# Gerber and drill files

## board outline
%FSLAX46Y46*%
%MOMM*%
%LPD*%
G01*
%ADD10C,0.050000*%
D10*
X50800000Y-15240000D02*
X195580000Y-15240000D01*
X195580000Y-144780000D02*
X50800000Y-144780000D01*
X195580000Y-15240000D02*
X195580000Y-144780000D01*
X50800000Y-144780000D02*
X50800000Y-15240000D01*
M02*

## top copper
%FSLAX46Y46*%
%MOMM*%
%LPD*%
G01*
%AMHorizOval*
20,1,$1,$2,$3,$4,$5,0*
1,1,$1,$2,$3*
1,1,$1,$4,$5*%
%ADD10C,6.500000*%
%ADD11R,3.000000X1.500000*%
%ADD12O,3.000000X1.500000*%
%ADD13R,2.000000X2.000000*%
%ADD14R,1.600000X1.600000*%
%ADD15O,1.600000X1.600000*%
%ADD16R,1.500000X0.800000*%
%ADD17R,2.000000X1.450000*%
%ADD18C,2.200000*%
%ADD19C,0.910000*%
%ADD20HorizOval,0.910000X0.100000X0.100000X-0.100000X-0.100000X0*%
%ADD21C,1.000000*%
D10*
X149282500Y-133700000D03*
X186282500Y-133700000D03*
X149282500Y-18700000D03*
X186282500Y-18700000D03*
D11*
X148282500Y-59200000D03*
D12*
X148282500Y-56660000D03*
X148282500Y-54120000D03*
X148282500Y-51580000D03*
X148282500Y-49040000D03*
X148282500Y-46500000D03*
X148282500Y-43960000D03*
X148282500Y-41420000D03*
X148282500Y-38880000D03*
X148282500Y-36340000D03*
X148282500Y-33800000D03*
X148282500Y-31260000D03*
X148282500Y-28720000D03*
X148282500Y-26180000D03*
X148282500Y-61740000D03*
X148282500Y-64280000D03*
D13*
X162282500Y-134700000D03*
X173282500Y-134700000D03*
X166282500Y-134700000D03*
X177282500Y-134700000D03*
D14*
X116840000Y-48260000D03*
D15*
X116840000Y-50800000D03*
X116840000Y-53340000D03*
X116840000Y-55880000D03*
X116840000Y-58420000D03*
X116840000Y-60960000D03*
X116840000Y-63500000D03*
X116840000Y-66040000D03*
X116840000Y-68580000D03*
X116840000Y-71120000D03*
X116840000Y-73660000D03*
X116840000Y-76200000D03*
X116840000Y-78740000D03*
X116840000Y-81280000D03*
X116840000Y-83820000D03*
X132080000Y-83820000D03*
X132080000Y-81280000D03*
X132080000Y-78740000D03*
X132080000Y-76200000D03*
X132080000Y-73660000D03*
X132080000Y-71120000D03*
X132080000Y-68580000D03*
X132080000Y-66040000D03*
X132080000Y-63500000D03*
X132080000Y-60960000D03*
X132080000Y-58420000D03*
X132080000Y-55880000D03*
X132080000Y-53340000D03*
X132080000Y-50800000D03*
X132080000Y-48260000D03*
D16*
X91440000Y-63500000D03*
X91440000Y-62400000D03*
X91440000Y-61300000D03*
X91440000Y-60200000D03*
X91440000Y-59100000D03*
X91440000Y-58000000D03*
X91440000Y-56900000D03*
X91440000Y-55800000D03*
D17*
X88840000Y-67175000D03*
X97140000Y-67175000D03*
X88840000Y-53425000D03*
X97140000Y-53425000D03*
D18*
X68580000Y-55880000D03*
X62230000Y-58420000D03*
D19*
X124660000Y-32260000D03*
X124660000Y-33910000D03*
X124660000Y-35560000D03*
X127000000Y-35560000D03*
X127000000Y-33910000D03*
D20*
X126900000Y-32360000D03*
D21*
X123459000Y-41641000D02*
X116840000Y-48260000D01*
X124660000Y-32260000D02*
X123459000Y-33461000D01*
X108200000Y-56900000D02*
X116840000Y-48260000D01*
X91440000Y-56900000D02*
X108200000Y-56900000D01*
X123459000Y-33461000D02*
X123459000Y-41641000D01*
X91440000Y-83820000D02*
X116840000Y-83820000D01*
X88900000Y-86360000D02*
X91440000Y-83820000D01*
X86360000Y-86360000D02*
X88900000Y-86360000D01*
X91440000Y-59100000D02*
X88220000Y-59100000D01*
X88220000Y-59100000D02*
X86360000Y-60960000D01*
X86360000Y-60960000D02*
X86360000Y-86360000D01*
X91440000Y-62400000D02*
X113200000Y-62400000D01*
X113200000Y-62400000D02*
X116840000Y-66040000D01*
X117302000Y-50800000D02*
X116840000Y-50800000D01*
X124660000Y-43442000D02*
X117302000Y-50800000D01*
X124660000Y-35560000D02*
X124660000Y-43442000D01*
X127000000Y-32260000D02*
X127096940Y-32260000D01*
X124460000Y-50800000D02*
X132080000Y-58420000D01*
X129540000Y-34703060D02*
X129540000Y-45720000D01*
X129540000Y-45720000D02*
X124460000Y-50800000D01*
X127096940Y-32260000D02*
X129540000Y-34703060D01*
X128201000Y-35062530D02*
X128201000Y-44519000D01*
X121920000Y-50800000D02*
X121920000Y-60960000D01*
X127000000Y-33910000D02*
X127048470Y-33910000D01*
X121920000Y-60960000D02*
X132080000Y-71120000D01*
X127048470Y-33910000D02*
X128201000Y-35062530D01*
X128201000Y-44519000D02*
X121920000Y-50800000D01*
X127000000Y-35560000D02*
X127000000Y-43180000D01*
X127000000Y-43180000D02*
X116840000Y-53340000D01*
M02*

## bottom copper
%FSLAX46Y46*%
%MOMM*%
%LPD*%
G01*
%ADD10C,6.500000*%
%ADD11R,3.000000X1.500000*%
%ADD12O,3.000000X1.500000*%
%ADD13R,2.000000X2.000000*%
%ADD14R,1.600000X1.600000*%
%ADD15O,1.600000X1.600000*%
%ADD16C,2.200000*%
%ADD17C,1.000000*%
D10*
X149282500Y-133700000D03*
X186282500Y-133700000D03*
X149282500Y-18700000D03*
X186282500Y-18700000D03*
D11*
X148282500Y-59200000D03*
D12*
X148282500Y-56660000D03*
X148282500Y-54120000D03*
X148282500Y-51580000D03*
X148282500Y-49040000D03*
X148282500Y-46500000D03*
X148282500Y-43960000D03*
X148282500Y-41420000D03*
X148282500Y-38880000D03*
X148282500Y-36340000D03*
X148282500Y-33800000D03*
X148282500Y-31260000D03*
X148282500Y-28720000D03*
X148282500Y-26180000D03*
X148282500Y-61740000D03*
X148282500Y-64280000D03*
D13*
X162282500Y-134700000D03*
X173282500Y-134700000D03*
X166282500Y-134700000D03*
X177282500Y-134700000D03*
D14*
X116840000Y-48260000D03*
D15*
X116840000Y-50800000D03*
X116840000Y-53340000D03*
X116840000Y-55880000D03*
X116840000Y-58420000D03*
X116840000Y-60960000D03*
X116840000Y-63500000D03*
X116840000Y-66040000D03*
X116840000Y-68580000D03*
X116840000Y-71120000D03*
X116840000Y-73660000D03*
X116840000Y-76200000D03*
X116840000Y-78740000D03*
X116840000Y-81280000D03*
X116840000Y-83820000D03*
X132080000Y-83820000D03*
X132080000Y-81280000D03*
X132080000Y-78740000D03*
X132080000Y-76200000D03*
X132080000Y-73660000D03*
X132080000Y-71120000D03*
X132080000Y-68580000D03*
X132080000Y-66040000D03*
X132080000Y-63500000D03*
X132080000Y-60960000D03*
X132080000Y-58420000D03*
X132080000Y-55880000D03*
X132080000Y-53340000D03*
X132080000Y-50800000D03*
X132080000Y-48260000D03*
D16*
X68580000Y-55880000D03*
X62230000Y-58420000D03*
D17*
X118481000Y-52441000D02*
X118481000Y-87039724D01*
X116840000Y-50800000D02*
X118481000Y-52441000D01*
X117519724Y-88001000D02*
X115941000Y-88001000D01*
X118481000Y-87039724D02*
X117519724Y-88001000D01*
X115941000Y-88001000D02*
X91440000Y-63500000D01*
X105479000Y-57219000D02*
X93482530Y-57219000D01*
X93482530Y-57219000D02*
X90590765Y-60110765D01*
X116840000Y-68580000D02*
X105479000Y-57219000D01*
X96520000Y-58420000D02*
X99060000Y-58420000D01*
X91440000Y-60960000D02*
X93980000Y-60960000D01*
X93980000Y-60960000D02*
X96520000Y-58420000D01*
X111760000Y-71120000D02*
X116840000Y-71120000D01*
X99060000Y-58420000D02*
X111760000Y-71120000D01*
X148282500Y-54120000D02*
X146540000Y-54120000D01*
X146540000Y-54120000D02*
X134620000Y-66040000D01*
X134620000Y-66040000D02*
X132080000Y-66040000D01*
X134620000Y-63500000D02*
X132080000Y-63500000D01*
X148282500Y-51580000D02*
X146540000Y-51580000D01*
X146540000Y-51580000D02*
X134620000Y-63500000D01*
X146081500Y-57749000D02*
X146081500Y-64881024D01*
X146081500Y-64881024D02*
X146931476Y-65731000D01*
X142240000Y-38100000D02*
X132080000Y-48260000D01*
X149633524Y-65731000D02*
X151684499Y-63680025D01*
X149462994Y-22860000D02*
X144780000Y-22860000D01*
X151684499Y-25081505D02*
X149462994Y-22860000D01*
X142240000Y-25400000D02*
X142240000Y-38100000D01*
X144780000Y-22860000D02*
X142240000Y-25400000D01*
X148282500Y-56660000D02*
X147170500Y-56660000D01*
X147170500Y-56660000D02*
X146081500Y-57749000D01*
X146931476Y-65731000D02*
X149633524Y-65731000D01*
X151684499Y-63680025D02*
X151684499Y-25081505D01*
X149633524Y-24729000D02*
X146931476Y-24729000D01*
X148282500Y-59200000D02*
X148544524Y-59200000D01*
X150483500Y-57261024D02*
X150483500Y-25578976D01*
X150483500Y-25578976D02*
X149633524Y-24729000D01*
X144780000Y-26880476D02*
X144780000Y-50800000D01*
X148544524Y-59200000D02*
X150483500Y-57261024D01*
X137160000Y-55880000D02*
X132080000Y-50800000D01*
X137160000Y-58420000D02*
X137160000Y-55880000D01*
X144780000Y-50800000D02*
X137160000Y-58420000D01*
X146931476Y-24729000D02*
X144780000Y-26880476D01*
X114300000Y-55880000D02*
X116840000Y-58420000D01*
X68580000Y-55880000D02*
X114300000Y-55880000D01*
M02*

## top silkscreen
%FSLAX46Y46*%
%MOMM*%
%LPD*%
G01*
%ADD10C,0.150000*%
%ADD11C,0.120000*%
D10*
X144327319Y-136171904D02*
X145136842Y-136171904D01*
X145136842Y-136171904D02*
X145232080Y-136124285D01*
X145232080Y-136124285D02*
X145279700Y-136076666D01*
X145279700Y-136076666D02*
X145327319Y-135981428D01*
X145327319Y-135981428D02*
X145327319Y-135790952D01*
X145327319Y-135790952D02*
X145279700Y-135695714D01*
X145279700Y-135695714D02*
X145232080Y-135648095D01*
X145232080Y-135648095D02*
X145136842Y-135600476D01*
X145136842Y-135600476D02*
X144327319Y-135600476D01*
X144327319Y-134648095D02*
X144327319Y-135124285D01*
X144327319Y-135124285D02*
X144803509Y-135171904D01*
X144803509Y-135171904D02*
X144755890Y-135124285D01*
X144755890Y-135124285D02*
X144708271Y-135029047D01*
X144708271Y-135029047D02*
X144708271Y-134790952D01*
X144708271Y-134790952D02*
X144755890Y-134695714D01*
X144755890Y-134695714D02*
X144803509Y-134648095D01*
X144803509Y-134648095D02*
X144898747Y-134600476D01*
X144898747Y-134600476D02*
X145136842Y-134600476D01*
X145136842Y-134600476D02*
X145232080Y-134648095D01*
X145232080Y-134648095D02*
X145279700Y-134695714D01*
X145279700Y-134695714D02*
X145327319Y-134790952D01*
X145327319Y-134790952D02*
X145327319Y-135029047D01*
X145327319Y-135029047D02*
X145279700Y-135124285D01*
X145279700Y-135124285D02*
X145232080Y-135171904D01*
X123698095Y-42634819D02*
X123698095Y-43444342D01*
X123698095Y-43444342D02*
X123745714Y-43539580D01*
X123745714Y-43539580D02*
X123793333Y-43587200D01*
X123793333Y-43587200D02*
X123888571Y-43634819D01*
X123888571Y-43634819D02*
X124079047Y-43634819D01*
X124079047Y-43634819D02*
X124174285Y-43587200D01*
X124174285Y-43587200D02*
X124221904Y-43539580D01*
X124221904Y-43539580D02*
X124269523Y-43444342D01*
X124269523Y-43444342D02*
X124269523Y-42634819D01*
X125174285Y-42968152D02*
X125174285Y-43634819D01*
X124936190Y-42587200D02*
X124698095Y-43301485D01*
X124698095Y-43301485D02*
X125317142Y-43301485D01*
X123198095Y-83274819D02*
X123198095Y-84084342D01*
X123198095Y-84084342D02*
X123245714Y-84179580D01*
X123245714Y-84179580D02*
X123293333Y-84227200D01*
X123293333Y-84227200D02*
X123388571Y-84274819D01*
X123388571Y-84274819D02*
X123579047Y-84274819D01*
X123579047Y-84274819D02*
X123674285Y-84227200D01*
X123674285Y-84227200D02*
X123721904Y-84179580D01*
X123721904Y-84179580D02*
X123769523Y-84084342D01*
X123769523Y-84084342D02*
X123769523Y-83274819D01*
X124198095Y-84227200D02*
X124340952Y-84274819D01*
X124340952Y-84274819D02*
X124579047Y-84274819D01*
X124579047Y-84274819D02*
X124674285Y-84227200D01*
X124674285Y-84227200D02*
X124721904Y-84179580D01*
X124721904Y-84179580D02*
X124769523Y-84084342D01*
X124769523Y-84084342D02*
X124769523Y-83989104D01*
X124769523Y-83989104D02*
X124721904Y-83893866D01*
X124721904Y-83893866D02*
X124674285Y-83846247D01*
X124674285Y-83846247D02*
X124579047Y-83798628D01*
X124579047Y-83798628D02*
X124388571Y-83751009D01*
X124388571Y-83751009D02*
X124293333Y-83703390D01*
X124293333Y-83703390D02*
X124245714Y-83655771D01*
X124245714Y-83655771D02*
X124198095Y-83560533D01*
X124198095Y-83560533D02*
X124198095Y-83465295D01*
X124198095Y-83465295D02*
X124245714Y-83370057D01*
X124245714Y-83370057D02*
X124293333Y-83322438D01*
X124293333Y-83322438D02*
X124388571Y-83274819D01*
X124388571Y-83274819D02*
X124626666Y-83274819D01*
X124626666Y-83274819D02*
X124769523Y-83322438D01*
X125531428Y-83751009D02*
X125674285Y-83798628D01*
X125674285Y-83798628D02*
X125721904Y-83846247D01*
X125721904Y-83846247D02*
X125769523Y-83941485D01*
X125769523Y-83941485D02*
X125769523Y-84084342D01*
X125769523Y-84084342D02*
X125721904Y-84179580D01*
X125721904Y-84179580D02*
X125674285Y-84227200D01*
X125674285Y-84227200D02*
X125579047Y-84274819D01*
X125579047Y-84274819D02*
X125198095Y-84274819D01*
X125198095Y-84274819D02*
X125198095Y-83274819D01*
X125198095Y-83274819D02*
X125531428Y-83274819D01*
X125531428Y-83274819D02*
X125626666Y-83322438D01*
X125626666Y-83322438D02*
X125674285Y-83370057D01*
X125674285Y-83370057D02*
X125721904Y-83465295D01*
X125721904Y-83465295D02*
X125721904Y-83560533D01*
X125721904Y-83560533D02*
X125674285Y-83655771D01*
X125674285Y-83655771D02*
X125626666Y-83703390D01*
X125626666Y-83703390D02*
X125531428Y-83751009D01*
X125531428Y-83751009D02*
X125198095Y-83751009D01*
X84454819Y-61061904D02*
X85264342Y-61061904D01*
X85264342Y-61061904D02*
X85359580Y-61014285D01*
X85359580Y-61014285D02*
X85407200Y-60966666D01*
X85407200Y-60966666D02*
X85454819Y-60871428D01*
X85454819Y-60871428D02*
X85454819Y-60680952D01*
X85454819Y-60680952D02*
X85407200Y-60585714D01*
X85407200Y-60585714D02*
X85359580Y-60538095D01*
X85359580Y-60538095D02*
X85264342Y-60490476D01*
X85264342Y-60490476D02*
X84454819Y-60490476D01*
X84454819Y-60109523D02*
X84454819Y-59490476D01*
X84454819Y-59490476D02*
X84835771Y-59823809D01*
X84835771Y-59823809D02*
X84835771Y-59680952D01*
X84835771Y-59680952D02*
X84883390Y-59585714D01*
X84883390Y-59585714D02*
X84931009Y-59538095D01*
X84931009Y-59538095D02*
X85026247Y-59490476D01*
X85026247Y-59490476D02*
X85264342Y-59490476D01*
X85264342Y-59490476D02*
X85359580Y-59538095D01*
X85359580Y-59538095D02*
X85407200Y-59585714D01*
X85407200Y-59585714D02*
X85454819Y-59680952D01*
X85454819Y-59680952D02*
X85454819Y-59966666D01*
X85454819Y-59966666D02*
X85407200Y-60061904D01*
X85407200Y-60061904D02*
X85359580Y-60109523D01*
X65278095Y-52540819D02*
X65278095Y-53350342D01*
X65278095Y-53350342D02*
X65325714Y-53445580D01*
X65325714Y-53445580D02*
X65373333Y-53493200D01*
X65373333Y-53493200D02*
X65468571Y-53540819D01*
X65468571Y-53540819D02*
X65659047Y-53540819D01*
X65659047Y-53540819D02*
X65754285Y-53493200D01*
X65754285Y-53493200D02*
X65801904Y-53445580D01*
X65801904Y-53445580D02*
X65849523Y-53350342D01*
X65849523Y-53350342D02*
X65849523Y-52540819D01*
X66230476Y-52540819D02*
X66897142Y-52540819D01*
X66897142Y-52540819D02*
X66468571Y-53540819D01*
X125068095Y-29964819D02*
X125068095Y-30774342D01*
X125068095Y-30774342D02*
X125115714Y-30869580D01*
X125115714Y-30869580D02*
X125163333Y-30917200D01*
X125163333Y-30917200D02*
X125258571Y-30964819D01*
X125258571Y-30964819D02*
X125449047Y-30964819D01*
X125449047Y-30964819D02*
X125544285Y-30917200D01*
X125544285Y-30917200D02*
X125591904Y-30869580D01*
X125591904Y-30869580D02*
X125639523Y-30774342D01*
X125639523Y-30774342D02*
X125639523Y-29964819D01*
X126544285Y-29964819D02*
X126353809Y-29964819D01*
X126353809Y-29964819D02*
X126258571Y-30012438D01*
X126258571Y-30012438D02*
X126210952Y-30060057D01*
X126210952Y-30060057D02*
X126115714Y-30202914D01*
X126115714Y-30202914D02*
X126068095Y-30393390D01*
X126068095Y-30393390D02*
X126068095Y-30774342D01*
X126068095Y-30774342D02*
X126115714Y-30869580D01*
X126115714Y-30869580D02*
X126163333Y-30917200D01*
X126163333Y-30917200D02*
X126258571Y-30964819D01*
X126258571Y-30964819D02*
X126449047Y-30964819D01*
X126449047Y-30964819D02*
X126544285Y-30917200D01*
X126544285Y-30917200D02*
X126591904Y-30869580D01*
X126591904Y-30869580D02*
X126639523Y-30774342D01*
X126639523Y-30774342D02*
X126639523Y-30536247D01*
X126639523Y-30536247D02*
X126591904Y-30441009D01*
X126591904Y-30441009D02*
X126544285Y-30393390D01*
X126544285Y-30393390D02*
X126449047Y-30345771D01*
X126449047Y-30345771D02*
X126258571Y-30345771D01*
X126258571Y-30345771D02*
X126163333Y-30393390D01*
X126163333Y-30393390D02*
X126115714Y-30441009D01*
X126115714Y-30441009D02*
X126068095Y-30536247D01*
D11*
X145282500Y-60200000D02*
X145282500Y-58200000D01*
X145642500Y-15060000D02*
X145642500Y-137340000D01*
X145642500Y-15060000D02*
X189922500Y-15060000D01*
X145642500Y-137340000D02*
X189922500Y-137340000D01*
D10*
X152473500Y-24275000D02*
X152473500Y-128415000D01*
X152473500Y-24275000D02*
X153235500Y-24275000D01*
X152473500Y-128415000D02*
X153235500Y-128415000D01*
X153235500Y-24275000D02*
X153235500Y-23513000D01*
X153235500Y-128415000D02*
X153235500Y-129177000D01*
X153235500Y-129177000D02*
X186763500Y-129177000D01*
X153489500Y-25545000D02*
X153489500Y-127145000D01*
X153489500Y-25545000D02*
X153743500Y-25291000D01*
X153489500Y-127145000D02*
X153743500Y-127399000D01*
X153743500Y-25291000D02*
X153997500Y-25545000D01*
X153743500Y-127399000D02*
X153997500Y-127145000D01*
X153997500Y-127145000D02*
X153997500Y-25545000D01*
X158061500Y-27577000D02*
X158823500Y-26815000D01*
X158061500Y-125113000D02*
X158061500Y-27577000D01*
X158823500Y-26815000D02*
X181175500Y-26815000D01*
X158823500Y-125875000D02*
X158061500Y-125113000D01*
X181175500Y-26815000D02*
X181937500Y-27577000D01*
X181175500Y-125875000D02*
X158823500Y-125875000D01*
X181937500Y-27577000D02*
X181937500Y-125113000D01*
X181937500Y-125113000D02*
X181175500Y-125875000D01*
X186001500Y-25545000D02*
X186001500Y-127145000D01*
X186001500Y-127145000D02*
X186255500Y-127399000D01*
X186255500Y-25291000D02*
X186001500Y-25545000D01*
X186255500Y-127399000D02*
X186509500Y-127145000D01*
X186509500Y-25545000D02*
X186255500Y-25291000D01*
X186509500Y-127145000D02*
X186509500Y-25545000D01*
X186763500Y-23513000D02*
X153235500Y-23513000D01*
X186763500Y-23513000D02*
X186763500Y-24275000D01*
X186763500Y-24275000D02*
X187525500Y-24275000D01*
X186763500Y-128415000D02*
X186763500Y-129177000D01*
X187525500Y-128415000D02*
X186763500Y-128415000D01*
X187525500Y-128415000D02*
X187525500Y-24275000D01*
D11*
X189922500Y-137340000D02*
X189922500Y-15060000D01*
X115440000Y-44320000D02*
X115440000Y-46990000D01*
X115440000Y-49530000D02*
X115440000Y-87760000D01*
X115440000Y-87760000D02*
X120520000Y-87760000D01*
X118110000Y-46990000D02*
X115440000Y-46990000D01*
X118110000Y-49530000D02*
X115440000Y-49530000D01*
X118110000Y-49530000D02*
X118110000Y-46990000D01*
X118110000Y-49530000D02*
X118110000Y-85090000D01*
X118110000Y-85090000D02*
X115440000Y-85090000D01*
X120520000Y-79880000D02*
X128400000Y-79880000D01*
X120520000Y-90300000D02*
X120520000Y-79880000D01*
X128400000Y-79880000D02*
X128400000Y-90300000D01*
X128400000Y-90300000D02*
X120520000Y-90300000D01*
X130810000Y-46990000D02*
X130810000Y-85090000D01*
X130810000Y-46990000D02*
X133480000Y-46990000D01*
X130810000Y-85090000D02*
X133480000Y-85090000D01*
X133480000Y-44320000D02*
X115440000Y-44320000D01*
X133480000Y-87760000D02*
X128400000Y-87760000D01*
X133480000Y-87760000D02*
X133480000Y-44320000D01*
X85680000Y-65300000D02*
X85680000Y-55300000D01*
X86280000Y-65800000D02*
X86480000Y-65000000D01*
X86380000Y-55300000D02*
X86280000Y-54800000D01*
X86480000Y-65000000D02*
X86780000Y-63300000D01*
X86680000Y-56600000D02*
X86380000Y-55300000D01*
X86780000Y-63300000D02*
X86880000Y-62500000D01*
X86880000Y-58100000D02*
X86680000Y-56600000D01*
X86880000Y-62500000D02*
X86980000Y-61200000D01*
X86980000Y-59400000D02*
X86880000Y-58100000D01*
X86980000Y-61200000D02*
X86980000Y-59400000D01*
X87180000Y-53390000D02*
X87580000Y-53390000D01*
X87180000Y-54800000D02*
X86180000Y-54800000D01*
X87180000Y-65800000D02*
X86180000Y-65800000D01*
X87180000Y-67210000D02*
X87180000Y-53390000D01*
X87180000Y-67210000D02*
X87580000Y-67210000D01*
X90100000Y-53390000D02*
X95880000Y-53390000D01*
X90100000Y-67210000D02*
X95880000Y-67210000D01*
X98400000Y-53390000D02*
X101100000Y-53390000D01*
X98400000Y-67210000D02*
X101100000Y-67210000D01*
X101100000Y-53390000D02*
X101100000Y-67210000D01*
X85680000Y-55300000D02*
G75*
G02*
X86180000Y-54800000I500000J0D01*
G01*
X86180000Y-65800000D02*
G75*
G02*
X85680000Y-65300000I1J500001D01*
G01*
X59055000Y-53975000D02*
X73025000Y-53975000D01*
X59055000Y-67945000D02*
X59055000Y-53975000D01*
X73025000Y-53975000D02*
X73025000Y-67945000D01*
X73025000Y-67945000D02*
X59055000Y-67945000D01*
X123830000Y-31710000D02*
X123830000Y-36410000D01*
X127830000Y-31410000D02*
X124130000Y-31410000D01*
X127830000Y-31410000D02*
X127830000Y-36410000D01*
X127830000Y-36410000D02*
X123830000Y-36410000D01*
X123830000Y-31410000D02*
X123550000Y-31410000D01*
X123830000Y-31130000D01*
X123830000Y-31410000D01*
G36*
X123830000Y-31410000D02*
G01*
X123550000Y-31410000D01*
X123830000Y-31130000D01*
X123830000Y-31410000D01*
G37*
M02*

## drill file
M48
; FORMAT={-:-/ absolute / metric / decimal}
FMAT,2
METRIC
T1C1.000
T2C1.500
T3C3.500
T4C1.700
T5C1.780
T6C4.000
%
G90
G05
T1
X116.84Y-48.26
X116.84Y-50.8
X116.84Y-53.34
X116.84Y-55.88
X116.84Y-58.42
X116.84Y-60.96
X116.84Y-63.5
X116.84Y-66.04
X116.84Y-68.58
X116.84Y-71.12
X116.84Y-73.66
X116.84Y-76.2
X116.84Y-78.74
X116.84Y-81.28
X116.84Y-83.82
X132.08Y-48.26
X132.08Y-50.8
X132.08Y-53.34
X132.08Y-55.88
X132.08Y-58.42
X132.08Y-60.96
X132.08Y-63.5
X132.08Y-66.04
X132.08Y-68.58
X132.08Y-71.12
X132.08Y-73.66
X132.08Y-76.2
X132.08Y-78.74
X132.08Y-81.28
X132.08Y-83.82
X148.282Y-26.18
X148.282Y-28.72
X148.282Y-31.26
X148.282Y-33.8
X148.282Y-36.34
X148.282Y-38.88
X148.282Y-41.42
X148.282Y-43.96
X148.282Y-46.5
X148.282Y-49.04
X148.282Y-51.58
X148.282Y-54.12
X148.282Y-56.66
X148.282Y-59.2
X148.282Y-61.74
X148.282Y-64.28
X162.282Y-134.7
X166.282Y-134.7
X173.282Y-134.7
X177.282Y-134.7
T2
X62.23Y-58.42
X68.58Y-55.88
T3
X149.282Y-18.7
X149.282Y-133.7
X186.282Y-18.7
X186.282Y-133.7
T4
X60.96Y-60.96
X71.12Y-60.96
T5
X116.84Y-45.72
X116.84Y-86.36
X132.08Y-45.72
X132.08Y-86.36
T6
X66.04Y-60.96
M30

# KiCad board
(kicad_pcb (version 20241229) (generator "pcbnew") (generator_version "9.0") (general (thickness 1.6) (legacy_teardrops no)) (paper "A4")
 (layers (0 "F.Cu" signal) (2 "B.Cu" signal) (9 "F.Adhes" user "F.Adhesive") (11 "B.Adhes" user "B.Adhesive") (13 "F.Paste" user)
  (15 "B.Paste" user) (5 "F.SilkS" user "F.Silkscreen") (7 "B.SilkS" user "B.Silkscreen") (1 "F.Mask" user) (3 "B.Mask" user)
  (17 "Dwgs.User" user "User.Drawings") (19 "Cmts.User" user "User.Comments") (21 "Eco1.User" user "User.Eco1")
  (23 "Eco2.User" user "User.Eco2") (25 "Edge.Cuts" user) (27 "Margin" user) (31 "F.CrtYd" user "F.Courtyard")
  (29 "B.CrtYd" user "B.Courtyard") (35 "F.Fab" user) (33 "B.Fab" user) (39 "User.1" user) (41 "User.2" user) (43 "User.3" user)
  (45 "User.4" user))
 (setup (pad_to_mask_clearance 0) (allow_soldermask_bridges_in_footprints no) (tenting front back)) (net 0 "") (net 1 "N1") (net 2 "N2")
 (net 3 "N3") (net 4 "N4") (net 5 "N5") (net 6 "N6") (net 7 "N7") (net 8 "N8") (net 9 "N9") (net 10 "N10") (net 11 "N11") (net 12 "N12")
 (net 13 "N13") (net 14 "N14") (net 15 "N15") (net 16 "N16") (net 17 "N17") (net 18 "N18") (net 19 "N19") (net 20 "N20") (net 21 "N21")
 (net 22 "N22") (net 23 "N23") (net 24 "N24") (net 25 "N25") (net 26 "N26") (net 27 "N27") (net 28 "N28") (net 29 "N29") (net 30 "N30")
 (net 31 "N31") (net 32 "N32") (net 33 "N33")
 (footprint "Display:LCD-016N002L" (layer "F.Cu") (at 148.2825 59.2 90)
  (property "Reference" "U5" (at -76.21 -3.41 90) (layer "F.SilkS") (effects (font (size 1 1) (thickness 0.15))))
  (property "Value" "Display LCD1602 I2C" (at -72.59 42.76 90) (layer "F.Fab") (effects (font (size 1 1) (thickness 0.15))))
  (fp_line (start -1 -3) (end 1 -3) (stroke (width 0.12) (type solid)) (layer "F.SilkS"))
  (fp_line (start 44.14 -2.64) (end -78.14 -2.64) (stroke (width 0.12) (type solid)) (layer "F.SilkS"))
  (fp_line (start 44.14 -2.64) (end 44.14 41.64) (stroke (width 0.12) (type solid)) (layer "F.SilkS"))
  (fp_line (start -78.14 -2.64) (end -78.14 41.64) (stroke (width 0.12) (type solid)) (layer "F.SilkS"))
  (fp_line (start 34.925 4.191) (end -69.215 4.191) (stroke (width 0.15) (type solid)) (layer "F.SilkS"))
  (fp_line (start 34.925 4.191) (end 34.925 4.953) (stroke (width 0.15) (type solid)) (layer "F.SilkS"))
  (fp_line (start -69.215 4.191) (end -69.215 4.953) (stroke (width 0.15) (type solid)) (layer "F.SilkS"))
  (fp_line (start 34.925 4.953) (end 35.687 4.953) (stroke (width 0.15) (type solid)) (layer "F.SilkS"))
  (fp_line (start -69.215 4.953) (end -69.977 4.953) (stroke (width 0.15) (type solid)) (layer "F.SilkS"))
  (fp_line (start -69.977 4.953) (end -69.977 38.481) (stroke (width 0.15) (type solid)) (layer "F.SilkS"))
  (fp_line (start 33.655 5.207) (end -67.945 5.207) (stroke (width 0.15) (type solid)) (layer "F.SilkS"))
  (fp_line (start 33.655 5.207) (end 33.909 5.461) (stroke (width 0.15) (type solid)) (layer "F.SilkS"))
  (fp_line (start -67.945 5.207) (end -68.199 5.461) (stroke (width 0.15) (type solid)) (layer "F.SilkS"))
  (fp_line (start 33.909 5.461) (end 33.655 5.715) (stroke (width 0.15) (type solid)) (layer "F.SilkS"))
  (fp_line (start -68.199 5.461) (end -67.945 5.715) (stroke (width 0.15) (type solid)) (layer "F.SilkS"))
  (fp_line (start -67.945 5.715) (end 33.655 5.715) (stroke (width 0.15) (type solid)) (layer "F.SilkS"))
  (fp_line (start 31.623 9.779) (end 32.385 10.541) (stroke (width 0.15) (type solid)) (layer "F.SilkS"))
  (fp_line (start -65.913 9.779) (end 31.623 9.779) (stroke (width 0.15) (type solid)) (layer "F.SilkS"))
  (fp_line (start 32.385 10.541) (end 32.385 32.893) (stroke (width 0.15) (type solid)) (layer "F.SilkS"))
  (fp_line (start -66.675 10.541) (end -65.913 9.779) (stroke (width 0.15) (type solid)) (layer "F.SilkS"))
  (fp_line (start 32.385 32.893) (end 31.623 33.655) (stroke (width 0.15) (type solid)) (layer "F.SilkS"))
  (fp_line (start -66.675 32.893) (end -66.675 10.541) (stroke (width 0.15) (type solid)) (layer "F.SilkS"))
  (fp_line (start 31.623 33.655) (end -65.913 33.655) (stroke (width 0.15) (type solid)) (layer "F.SilkS"))
  (fp_line (start -65.913 33.655) (end -66.675 32.893) (stroke (width 0.15) (type solid)) (layer "F.SilkS"))
  (fp_line (start 33.655 37.719) (end -67.945 37.719) (stroke (width 0.15) (type solid)) (layer "F.SilkS"))
  (fp_line (start -67.945 37.719) (end -68.199 37.973) (stroke (width 0.15) (type solid)) (layer "F.SilkS"))
  (fp_line (start 33.909 37.973) (end 33.655 37.719) (stroke (width 0.15) (type solid)) (layer "F.SilkS"))
  (fp_line (start -68.199 37.973) (end -67.945 38.227) (stroke (width 0.15) (type solid)) (layer "F.SilkS"))
  (fp_line (start 33.655 38.227) (end 33.909 37.973) (stroke (width 0.15) (type solid)) (layer "F.SilkS"))
  (fp_line (start -67.945 38.227) (end 33.655 38.227) (stroke (width 0.15) (type solid)) (layer "F.SilkS"))
  (fp_line (start 35.687 38.481) (end 35.687 4.953) (stroke (width 0.15) (type solid)) (layer "F.SilkS"))
  (fp_line (start 35.687 38.481) (end 34.925 38.481) (stroke (width 0.15) (type solid)) (layer "F.SilkS"))
  (fp_line (start 34.925 38.481) (end 34.925 39.243) (stroke (width 0.15) (type solid)) (layer "F.SilkS"))
  (fp_line (start -69.215 38.481) (end -69.977 38.481) (stroke (width 0.15) (type solid)) (layer "F.SilkS"))
  (fp_line (start -69.215 39.243) (end -69.215 38.481) (stroke (width 0.15) (type solid)) (layer "F.SilkS"))
  (fp_line (start -69.215 39.243) (end 34.925 39.243) (stroke (width 0.15) (type solid)) (layer "F.SilkS"))
  (fp_line (start -78.14 41.64) (end 44.14 41.64) (stroke (width 0.12) (type solid)) (layer "F.SilkS"))
  (pad "" thru_hole circle (at -74.5 1 270) (size 6.5 6.5) (drill 3.5) (layers "*.Cu" "*.Mask") (remove_unused_layers no))
  (pad "" thru_hole circle (at -74.5 38 270) (size 6.5 6.5) (drill 3.5) (layers "*.Cu" "*.Mask") (remove_unused_layers no))
  (pad "" thru_hole circle (at 40.5 1 270) (size 6.5 6.5) (drill 3.5) (layers "*.Cu" "*.Mask") (remove_unused_layers no))
  (pad "" thru_hole circle (at 40.5 38 270) (size 6.5 6.5) (drill 3.5) (layers "*.Cu" "*.Mask") (remove_unused_layers no))
  (pad "1" thru_hole rect (at 0 0 270) (size 1.5 3) (drill 1) (layers "*.Cu" "*.Mask") (remove_unused_layers no) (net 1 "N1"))
  (pad "2" thru_hole oval (at 2.54 0 270) (size 1.5 3) (drill 1) (layers "*.Cu" "*.Mask") (remove_unused_layers no) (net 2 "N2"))
  (pad "3" thru_hole oval (at 5.08 0 270) (size 1.5 3) (drill 1) (layers "*.Cu" "*.Mask") (remove_unused_layers no) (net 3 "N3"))
  (pad "4" thru_hole oval (at 7.62 0 270) (size 1.5 3) (drill 1) (layers "*.Cu" "*.Mask") (remove_unused_layers no) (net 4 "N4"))
  (pad "5" thru_hole oval (at 10.16 0 270) (size 1.5 3) (drill 1) (layers "*.Cu" "*.Mask") (remove_unused_layers no))
  (pad "6" thru_hole oval (at 12.7 0 270) (size 1.5 3) (drill 1) (layers "*.Cu" "*.Mask") (remove_unused_layers no))
  (pad "7" thru_hole oval (at 15.24 0 270) (size 1.5 3) (drill 1) (layers "*.Cu" "*.Mask") (remove_unused_layers no))
  (pad "8" thru_hole oval (at 17.78 0 270) (size 1.5 3) (drill 1) (layers "*.Cu" "*.Mask") (remove_unused_layers no))
  (pad "9" thru_hole oval (at 20.32 0 270) (size 1.5 3) (drill 1) (layers "*.Cu" "*.Mask") (remove_unused_layers no))
  (pad "10" thru_hole oval (at 22.86 0 270) (size 1.5 3) (drill 1) (layers "*.Cu" "*.Mask") (remove_unused_layers no))
  (pad "11" thru_hole oval (at 25.4 0 270) (size 1.5 3) (drill 1) (layers "*.Cu" "*.Mask") (remove_unused_layers no))
  (pad "12" thru_hole oval (at 27.94 0 270) (size 1.5 3) (drill 1) (layers "*.Cu" "*.Mask") (remove_unused_layers no))
  (pad "13" thru_hole oval (at 30.48 0 270) (size 1.5 3) (drill 1) (layers "*.Cu" "*.Mask") (remove_unused_layers no))
  (pad "14" thru_hole oval (at 33.02 0 270) (size 1.5 3) (drill 1) (layers "*.Cu" "*.Mask") (remove_unused_layers no))
  (pad "15" thru_hole oval (at -2.54 0 270) (size 1.5 3) (drill 1) (layers "*.Cu" "*.Mask") (remove_unused_layers no))
  (pad "16" thru_hole oval (at -5.08 0 270) (size 1.5 3) (drill 1) (layers "*.Cu" "*.Mask") (remove_unused_layers no))
  (pad "A1" thru_hole rect (at -75.5 14 270) (size 2 2) (drill 1) (layers "*.Cu" "*.Mask") (remove_unused_layers no))
  (pad "A2" thru_hole rect (at -75.5 25 270) (size 2 2) (drill 1) (layers "*.Cu" "*.Mask") (remove_unused_layers no))
  (pad "K1" thru_hole rect (at -75.5 18 270) (size 2 2) (drill 1) (layers "*.Cu" "*.Mask") (remove_unused_layers no))
  (pad "K2" thru_hole rect (at -75.5 29 270) (size 2 2) (drill 1) (layers "*.Cu" "*.Mask") (remove_unused_layers no)))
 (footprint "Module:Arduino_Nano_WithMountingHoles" (layer "F.Cu") (at 116.84 48.26)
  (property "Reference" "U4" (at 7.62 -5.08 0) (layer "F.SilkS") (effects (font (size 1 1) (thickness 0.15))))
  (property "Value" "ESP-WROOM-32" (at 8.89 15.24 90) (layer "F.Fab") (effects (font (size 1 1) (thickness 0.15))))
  (fp_line (start -1.4 -3.94) (end -1.4 -1.27) (stroke (width 0.12) (type solid)) (layer "F.SilkS"))
  (fp_line (start -1.4 1.27) (end -1.4 39.5) (stroke (width 0.12) (type solid)) (layer "F.SilkS"))
  (fp_line (start -1.4 39.5) (end 3.68 39.5) (stroke (width 0.12) (type solid)) (layer "F.SilkS"))
  (fp_line (start 1.27 -1.27) (end -1.4 -1.27) (stroke (width 0.12) (type solid)) (layer "F.SilkS"))
  (fp_line (start 1.27 1.27) (end -1.4 1.27) (stroke (width 0.12) (type solid)) (layer "F.SilkS"))
  (fp_line (start 1.27 1.27) (end 1.27 -1.27) (stroke (width 0.12) (type solid)) (layer "F.SilkS"))
  (fp_line (start 1.27 1.27) (end 1.27 36.83) (stroke (width 0.12) (type solid)) (layer "F.SilkS"))
  (fp_line (start 1.27 36.83) (end -1.4 36.83) (stroke (width 0.12) (type solid)) (layer "F.SilkS"))
  (fp_line (start 3.68 31.62) (end 11.56 31.62) (stroke (width 0.12) (type solid)) (layer "F.SilkS"))
  (fp_line (start 3.68 42.04) (end 3.68 31.62) (stroke (width 0.12) (type solid)) (layer "F.SilkS"))
  (fp_line (start 11.56 31.62) (end 11.56 42.04) (stroke (width 0.12) (type solid)) (layer "F.SilkS"))
  (fp_line (start 11.56 42.04) (end 3.68 42.04) (stroke (width 0.12) (type solid)) (layer "F.SilkS"))
  (fp_line (start 13.97 -1.27) (end 13.97 36.83) (stroke (width 0.12) (type solid)) (layer "F.SilkS"))
  (fp_line (start 13.97 -1.27) (end 16.64 -1.27) (stroke (width 0.12) (type solid)) (layer "F.SilkS"))
  (fp_line (start 13.97 36.83) (end 16.64 36.83) (stroke (width 0.12) (type solid)) (layer "F.SilkS"))
  (fp_line (start 16.64 -3.94) (end -1.4 -3.94) (stroke (width 0.12) (type solid)) (layer "F.SilkS"))
  (fp_line (start 16.64 39.5) (end 11.56 39.5) (stroke (width 0.12) (type solid)) (layer "F.SilkS"))
  (fp_line (start 16.64 39.5) (end 16.64 -3.94) (stroke (width 0.12) (type solid)) (layer "F.SilkS"))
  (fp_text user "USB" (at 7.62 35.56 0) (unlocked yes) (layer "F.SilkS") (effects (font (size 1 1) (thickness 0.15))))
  (pad "" np_thru_hole circle (at 0 -2.54) (size 1.78 1.78) (drill 1.78) (layers "*.Cu" "*.Mask"))
  (pad "" np_thru_hole circle (at 0 38.1) (size 1.78 1.78) (drill 1.78) (layers "*.Cu" "*.Mask"))
  (pad "" np_thru_hole circle (at 15.24 -2.54) (size 1.78 1.78) (drill 1.78) (layers "*.Cu" "*.Mask"))
  (pad "" np_thru_hole circle (at 15.24 38.1) (size 1.78 1.78) (drill 1.78) (layers "*.Cu" "*.Mask"))
  (pad "1" thru_hole rect (at 0 0) (size 1.6 1.6) (drill 1) (layers "*.Cu" "*.Mask") (remove_unused_layers no) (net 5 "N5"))
  (pad "2" thru_hole oval (at 0 2.54) (size 1.6 1.6) (drill 1) (layers "*.Cu" "*.Mask") (remove_unused_layers no) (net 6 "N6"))
  (pad "3" thru_hole oval (at 0 5.08) (size 1.6 1.6) (drill 1) (layers "*.Cu" "*.Mask") (remove_unused_layers no) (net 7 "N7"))
  (pad "4" thru_hole oval (at 0 7.62) (size 1.6 1.6) (drill 1) (layers "*.Cu" "*.Mask") (remove_unused_layers no) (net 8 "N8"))
  (pad "5" thru_hole oval (at 0 10.16) (size 1.6 1.6) (drill 1) (layers "*.Cu" "*.Mask") (remove_unused_layers no) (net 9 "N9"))
  (pad "6" thru_hole oval (at 0 12.7) (size 1.6 1.6) (drill 1) (layers "*.Cu" "*.Mask") (remove_unused_layers no) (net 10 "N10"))
  (pad "7" thru_hole oval (at 0 15.24) (size 1.6 1.6) (drill 1) (layers "*.Cu" "*.Mask") (remove_unused_layers no) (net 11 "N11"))
  (pad "8" thru_hole oval (at 0 17.78) (size 1.6 1.6) (drill 1) (layers "*.Cu" "*.Mask") (remove_unused_layers no) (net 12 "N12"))
  (pad "9" thru_hole oval (at 0 20.32) (size 1.6 1.6) (drill 1) (layers "*.Cu" "*.Mask") (remove_unused_layers no) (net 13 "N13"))
  (pad "10" thru_hole oval (at 0 22.86) (size 1.6 1.6) (drill 1) (layers "*.Cu" "*.Mask") (remove_unused_layers no) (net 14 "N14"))
  (pad "11" thru_hole oval (at 0 25.4) (size 1.6 1.6) (drill 1) (layers "*.Cu" "*.Mask") (remove_unused_layers no) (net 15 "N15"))
  (pad "12" thru_hole oval (at 0 27.94) (size 1.6 1.6) (drill 1) (layers "*.Cu" "*.Mask") (remove_unused_layers no) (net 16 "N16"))
  (pad "13" thru_hole oval (at 0 30.48) (size 1.6 1.6) (drill 1) (layers "*.Cu" "*.Mask") (remove_unused_layers no) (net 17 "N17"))
  (pad "14" thru_hole oval (at 0 33.02) (size 1.6 1.6) (drill 1) (layers "*.Cu" "*.Mask") (remove_unused_layers no) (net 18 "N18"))
  (pad "15" thru_hole oval (at 0 35.56) (size 1.6 1.6) (drill 1) (layers "*.Cu" "*.Mask") (remove_unused_layers no) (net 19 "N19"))
  (pad "16" thru_hole oval (at 15.24 35.56) (size 1.6 1.6) (drill 1) (layers "*.Cu" "*.Mask") (remove_unused_layers no) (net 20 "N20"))
  (pad "17" thru_hole oval (at 15.24 33.02) (size 1.6 1.6) (drill 1) (layers "*.Cu" "*.Mask") (remove_unused_layers no) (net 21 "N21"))
  (pad "18" thru_hole oval (at 15.24 30.48) (size 1.6 1.6) (drill 1) (layers "*.Cu" "*.Mask") (remove_unused_layers no) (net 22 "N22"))
  (pad "19" thru_hole oval (at 15.24 27.94) (size 1.6 1.6) (drill 1) (layers "*.Cu" "*.Mask") (remove_unused_layers no) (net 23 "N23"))
  (pad "20" thru_hole oval (at 15.24 25.4) (size 1.6 1.6) (drill 1) (layers "*.Cu" "*.Mask") (remove_unused_layers no) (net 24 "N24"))
  (pad "21" thru_hole oval (at 15.24 22.86) (size 1.6 1.6) (drill 1) (layers "*.Cu" "*.Mask") (remove_unused_layers no) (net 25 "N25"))
  (pad "22" thru_hole oval (at 15.24 20.32) (size 1.6 1.6) (drill 1) (layers "*.Cu" "*.Mask") (remove_unused_layers no) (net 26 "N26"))
  (pad "23" thru_hole oval (at 15.24 17.78) (size 1.6 1.6) (drill 1) (layers "*.Cu" "*.Mask") (remove_unused_layers no) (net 3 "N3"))
  (pad "24" thru_hole oval (at 15.24 15.24) (size 1.6 1.6) (drill 1) (layers "*.Cu" "*.Mask") (remove_unused_layers no) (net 4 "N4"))
  (pad "25" thru_hole oval (at 15.24 12.7) (size 1.6 1.6) (drill 1) (layers "*.Cu" "*.Mask") (remove_unused_layers no) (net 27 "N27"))
  (pad "26" thru_hole oval (at 15.24 10.16) (size 1.6 1.6) (drill 1) (layers "*.Cu" "*.Mask") (remove_unused_layers no) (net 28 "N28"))
  (pad "27" thru_hole oval (at 15.24 7.62) (size 1.6 1.6) (drill 1) (layers "*.Cu" "*.Mask") (remove_unused_layers no) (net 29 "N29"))
  (pad "28" thru_hole oval (at 15.24 5.08) (size 1.6 1.6) (drill 1) (layers "*.Cu" "*.Mask") (remove_unused_layers no) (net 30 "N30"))
  (pad "29" thru_hole oval (at 15.24 2.54) (size 1.6 1.6) (drill 1) (layers "*.Cu" "*.Mask") (remove_unused_layers no) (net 1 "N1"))
  (pad "30" thru_hole oval (at 15.24 0) (size 1.6 1.6) (drill 1) (layers "*.Cu" "*.Mask") (remove_unused_layers no) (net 2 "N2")))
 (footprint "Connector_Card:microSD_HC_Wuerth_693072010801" (layer "F.Cu") (at 92.99 60.3 90)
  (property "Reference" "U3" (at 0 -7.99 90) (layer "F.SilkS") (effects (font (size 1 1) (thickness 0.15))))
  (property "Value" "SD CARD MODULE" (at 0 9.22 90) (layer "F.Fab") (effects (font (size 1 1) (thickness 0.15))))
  (fp_line (start -5 -7.31) (end 5 -7.31) (stroke (width 0.12) (type solid)) (layer "F.SilkS"))
  (fp_line (start -5.5 -6.71) (end -4.7 -6.51) (stroke (width 0.12) (type solid)) (layer "F.SilkS"))
  (fp_line (start 5 -6.61) (end 5.5 -6.71) (stroke (width 0.12) (type solid)) (layer "F.SilkS"))
  (fp_line (start -4.7 -6.51) (end -3 -6.21) (stroke (width 0.12) (type solid)) (layer "F.SilkS"))
  (fp_line (start 3.7 -6.31) (end 5 -6.61) (stroke (width 0.12) (type solid)) (layer "F.SilkS"))
  (fp_line (start -3 -6.21) (end -2.2 -6.11) (stroke (width 0.12) (type solid)) (layer "F.SilkS"))
  (fp_line (start 2.2 -6.11) (end 3.7 -6.31) (stroke (width 0.12) (type solid)) (layer "F.SilkS"))
  (fp_line (start -2.2 -6.11) (end -0.9 -6.01) (stroke (width 0.12) (type solid)) (layer "F.SilkS"))
  (fp_line (start 0.9 -6.01) (end 2.2 -6.11) (stroke (width 0.12) (type solid)) (layer "F.SilkS"))
  (fp_line (start -0.9 -6.01) (end 0.9 -6.01) (stroke (width 0.12) (type solid)) (layer "F.SilkS"))
  (fp_line (start 6.91 -5.81) (end 6.91 -5.41) (stroke (width 0.12) (type solid)) (layer "F.SilkS"))
  (fp_line (start 5.5 -5.81) (end 5.5 -6.81) (stroke (width 0.12) (type solid)) (layer "F.SilkS"))
  (fp_line (start -5.5 -5.81) (end -5.5 -6.81) (stroke (width 0.12) (type solid)) (layer "F.SilkS"))
  (fp_line (start -6.91 -5.81) (end 6.91 -5.81) (stroke (width 0.12) (type solid)) (layer "F.SilkS"))
  (fp_line (start -6.91 -5.81) (end -6.91 -5.41) (stroke (width 0.12) (type solid)) (layer "F.SilkS"))
  (fp_line (start 6.91 -2.89) (end 6.91 2.89) (stroke (width 0.12) (type solid)) (layer "F.SilkS"))
  (fp_line (start -6.91 -2.89) (end -6.91 2.89) (stroke (width 0.12) (type solid)) (layer "F.SilkS"))
  (fp_line (start 6.91 5.41) (end 6.91 8.11) (stroke (width 0.12) (type solid)) (layer "F.SilkS"))
  (fp_line (start -6.91 5.41) (end -6.91 8.11) (stroke (width 0.12) (type solid)) (layer "F.SilkS"))
  (fp_line (start 6.91 8.11) (end -6.91 8.11) (stroke (width 0.12) (type solid)) (layer "F.SilkS"))
  (fp_arc (start 5 -7.31) (mid 5.353553 -7.163553) (end 5.5 -6.81) (stroke (width 0.12) (type solid)) (layer "F.SilkS"))
  (fp_arc (start -5.5 -6.81) (mid -5.353553 -7.163553) (end -5 -7.31) (stroke (width 0.12) (type solid)) (layer "F.SilkS"))
  (pad "1" smd rect (at -3.2 -1.55 90) (size 0.8 1.5) (layers "F.Cu" "F.Mask" "F.Paste") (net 6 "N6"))
  (pad "2" smd rect (at -2.1 -1.55 90) (size 0.8 1.5) (layers "F.Cu" "F.Mask" "F.Paste") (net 12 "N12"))
  (pad "3" smd rect (at -1 -1.55 90) (size 0.8 1.5) (layers "F.Cu" "F.Mask" "F.Paste") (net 13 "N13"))
  (pad "4" smd rect (at 0.1 -1.55 90) (size 0.8 1.5) (layers "F.Cu" "F.Mask" "F.Paste") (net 14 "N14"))
  (pad "5" smd rect (at 1.2 -1.55 90) (size 0.8 1.5) (layers "F.Cu" "F.Mask" "F.Paste") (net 19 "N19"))
  (pad "6" smd rect (at 2.3 -1.55 90) (size 0.8 1.5) (layers "F.Cu" "F.Mask" "F.Paste") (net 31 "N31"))
  (pad "7" smd rect (at 3.4 -1.55 90) (size 0.8 1.5) (layers "F.Cu" "F.Mask" "F.Paste") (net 5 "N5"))
  (pad "8" smd rect (at 4.5 -1.55 90) (size 0.8 1.5) (layers "F.Cu" "F.Mask" "F.Paste") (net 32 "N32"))
  (pad "9" smd rect (at -6.875 -4.15 90) (size 1.45 2) (layers "F.Cu" "F.Mask" "F.Paste"))
  (pad "9" smd rect (at -6.875 4.15 90) (size 1.45 2) (layers "F.Cu" "F.Mask" "F.Paste"))
  (pad "9" smd rect (at 6.875 -4.15 90) (size 1.45 2) (layers "F.Cu" "F.Mask" "F.Paste"))
  (pad "9" smd rect (at 6.875 4.15 90) (size 1.45 2) (layers "F.Cu" "F.Mask" "F.Paste")))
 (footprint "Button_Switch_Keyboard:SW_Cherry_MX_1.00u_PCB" (layer "F.Cu") (at 68.58 55.88)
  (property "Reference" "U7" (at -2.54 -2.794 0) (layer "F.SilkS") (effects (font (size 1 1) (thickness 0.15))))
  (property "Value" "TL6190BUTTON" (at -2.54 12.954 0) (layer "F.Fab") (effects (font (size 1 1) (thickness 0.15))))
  (fp_line (start -9.525 -1.905) (end 4.445 -1.905) (stroke (width 0.12) (type solid)) (layer "F.SilkS"))
  (fp_line (start -9.525 12.065) (end -9.525 -1.905) (stroke (width 0.12) (type solid)) (layer "F.SilkS"))
  (fp_line (start 4.445 -1.905) (end 4.445 12.065) (stroke (width 0.12) (type solid)) (layer "F.SilkS"))
  (fp_line (start 4.445 12.065) (end -9.525 12.065) (stroke (width 0.12) (type solid)) (layer "F.SilkS"))
  (pad "" np_thru_hole circle (at -7.62 5.08) (size 1.7 1.7) (drill 1.7) (layers "*.Cu" "*.Mask"))
  (pad "" np_thru_hole circle (at -2.54 5.08) (size 4 4) (drill 4) (layers "*.Cu" "*.Mask"))
  (pad "" np_thru_hole circle (at 2.54 5.08) (size 1.7 1.7) (drill 1.7) (layers "*.Cu" "*.Mask"))
  (pad "1" thru_hole circle (at 0 0) (size 2.2 2.2) (drill 1.5) (layers "*.Cu" "*.Mask") (remove_unused_layers no) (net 9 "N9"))
  (pad "2" thru_hole circle (at -6.35 2.54) (size 2.2 2.2) (drill 1.5) (layers "*.Cu" "*.Mask") (remove_unused_layers no) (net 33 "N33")))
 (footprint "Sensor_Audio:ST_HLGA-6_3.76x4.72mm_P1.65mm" (layer "F.Cu") (at 125.83 33.91)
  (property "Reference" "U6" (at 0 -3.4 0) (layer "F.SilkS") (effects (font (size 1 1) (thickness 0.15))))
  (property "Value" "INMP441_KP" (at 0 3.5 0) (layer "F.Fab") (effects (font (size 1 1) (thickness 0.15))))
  (fp_line (start -2 -2.2) (end -2 2.5) (stroke (width 0.12) (type solid)) (layer "F.SilkS"))
  (fp_line (start 2 -2.5) (end -1.7 -2.5) (stroke (width 0.12) (type solid)) (layer "F.SilkS"))
  (fp_line (start 2 -2.5) (end 2 2.5) (stroke (width 0.12) (type solid)) (layer "F.SilkS"))
  (fp_line (start 2 2.5) (end -2 2.5) (stroke (width 0.12) (type solid)) (layer "F.SilkS"))
  (fp_poly (pts (xy -2 -2.5) (xy -2.28 -2.5) (xy -2 -2.78) (xy -2 -2.5)) (stroke (width 0.12) (type solid)) (fill yes) (layer "F.SilkS"))
  (pad "1" smd circle (at -1.17 -1.65) (size 0.91 0.91) (layers "F.Cu" "F.Mask" "F.Paste") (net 5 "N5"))
  (pad "2" smd circle (at -1.17 0) (size 0.91 0.91) (layers "F.Cu" "F.Mask" "F.Paste") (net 6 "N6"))
  (pad "3" smd circle (at -1.17 1.65) (size 0.91 0.91) (layers "F.Cu" "F.Mask" "F.Paste") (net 6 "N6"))
  (pad "4" smd circle (at 1.17 1.65) (size 0.91 0.91) (layers "F.Cu" "F.Mask" "F.Paste") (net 7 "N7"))
  (pad "5" smd circle (at 1.17 0) (size 0.91 0.91) (layers "F.Cu" "F.Mask" "F.Paste") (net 25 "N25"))
  (pad "6" smd oval (at 1.17 -1.65 45) (size 1.192843 0.91) (drill (offset -0.141421 0)) (layers "F.Cu" "F.Mask" "F.Paste") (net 28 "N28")))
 (gr_line (start 50.8 15.24) (end 195.58 15.24) (stroke (width 0.05) (type default)) (layer "Edge.Cuts"))
 (gr_line (start 195.58 144.78) (end 50.8 144.78) (stroke (width 0.05) (type default)) (layer "Edge.Cuts"))
 (gr_line (start 195.58 15.24) (end 195.58 144.78) (stroke (width 0.05) (type default)) (layer "Edge.Cuts"))
 (gr_line (start 50.8 144.78) (end 50.8 15.24) (stroke (width 0.05) (type default)) (layer "Edge.Cuts"))
 (segment (start 123.459 41.641) (end 116.84 48.26) (width 1) (layer "F.Cu") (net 5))
 (segment (start 124.66 32.26) (end 123.459 33.461) (width 1) (layer "F.Cu") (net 5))
 (segment (start 108.2 56.9) (end 116.84 48.26) (width 1) (layer "F.Cu") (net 5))
 (segment (start 91.44 56.9) (end 108.2 56.9) (width 1) (layer "F.Cu") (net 5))
 (segment (start 123.459 33.461) (end 123.459 41.641) (width 1) (layer "F.Cu") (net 5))
 (segment (start 91.44 83.82) (end 116.84 83.82) (width 1) (layer "F.Cu") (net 19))
 (segment (start 88.9 86.36) (end 91.44 83.82) (width 1) (layer "F.Cu") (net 19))
 (segment (start 86.36 86.36) (end 88.9 86.36) (width 1) (layer "F.Cu") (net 19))
 (segment (start 91.44 59.1) (end 88.22 59.1) (width 1) (layer "F.Cu") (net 19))
 (segment (start 88.22 59.1) (end 86.36 60.96) (width 1) (layer "F.Cu") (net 19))
 (segment (start 86.36 60.96) (end 86.36 86.36) (width 1) (layer "F.Cu") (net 19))
 (segment (start 91.44 62.4) (end 113.2 62.4) (width 1) (layer "F.Cu") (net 12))
 (segment (start 113.2 62.4) (end 116.84 66.04) (width 1) (layer "F.Cu") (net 12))
 (segment (start 117.302 50.8) (end 116.84 50.8) (width 1) (layer "F.Cu") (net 6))
 (segment (start 124.66 43.442) (end 117.302 50.8) (width 1) (layer "F.Cu") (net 6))
 (segment (start 124.66 35.56) (end 124.66 43.442) (width 1) (layer "F.Cu") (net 6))
 (segment (start 118.481 52.441) (end 118.481 87.039724) (width 1) (layer "B.Cu") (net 6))
 (segment (start 116.84 50.8) (end 118.481 52.441) (width 1) (layer "B.Cu") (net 6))
 (segment (start 117.519724 88.001) (end 115.941 88.001) (width 1) (layer "B.Cu") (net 6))
 (segment (start 118.481 87.039724) (end 117.519724 88.001) (width 1) (layer "B.Cu") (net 6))
 (segment (start 115.941 88.001) (end 91.44 63.5) (width 1) (layer "B.Cu") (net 6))
 (segment (start 105.479 57.219) (end 93.48253 57.219) (width 1) (layer "B.Cu") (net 13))
 (segment (start 93.48253 57.219) (end 90.590765 60.110765) (width 1) (layer "B.Cu") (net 13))
 (segment (start 116.84 68.58) (end 105.479 57.219) (width 1) (layer "B.Cu") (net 13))
 (segment (start 96.52 58.42) (end 99.06 58.42) (width 1) (layer "B.Cu") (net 14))
 (segment (start 91.44 60.96) (end 93.98 60.96) (width 1) (layer "B.Cu") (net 14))
 (segment (start 93.98 60.96) (end 96.52 58.42) (width 1) (layer "B.Cu") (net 14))
 (segment (start 111.76 71.12) (end 116.84 71.12) (width 1) (layer "B.Cu") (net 14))
 (segment (start 99.06 58.42) (end 111.76 71.12) (width 1) (layer "B.Cu") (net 14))
 (segment (start 148.2825 54.12) (end 146.54 54.12) (width 1) (layer "B.Cu") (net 3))
 (segment (start 146.54 54.12) (end 134.62 66.04) (width 1) (layer "B.Cu") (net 3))
 (segment (start 134.62 66.04) (end 132.08 66.04) (width 1) (layer "B.Cu") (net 3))
 (segment (start 134.62 63.5) (end 132.08 63.5) (width 1) (layer "B.Cu") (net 4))
 (segment (start 148.2825 51.58) (end 146.54 51.58) (width 1) (layer "B.Cu") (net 4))
 (segment (start 146.54 51.58) (end 134.62 63.5) (width 1) (layer "B.Cu") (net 4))
 (segment (start 146.0815 57.749) (end 146.0815 64.881024) (width 1) (layer "B.Cu") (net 2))
 (segment (start 146.0815 64.881024) (end 146.931476 65.731) (width 1) (layer "B.Cu") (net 2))
 (segment (start 142.24 38.1) (end 132.08 48.26) (width 1) (layer "B.Cu") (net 2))
 (segment (start 149.633524 65.731) (end 151.684499 63.680025) (width 1) (layer "B.Cu") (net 2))
 (segment (start 149.462994 22.86) (end 144.78 22.86) (width 1) (layer "B.Cu") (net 2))
 (segment (start 151.684499 25.081505) (end 149.462994 22.86) (width 1) (layer "B.Cu") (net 2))
 (segment (start 142.24 25.4) (end 142.24 38.1) (width 1) (layer "B.Cu") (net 2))
 (segment (start 144.78 22.86) (end 142.24 25.4) (width 1) (layer "B.Cu") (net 2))
 (segment (start 148.2825 56.66) (end 147.1705 56.66) (width 1) (layer "B.Cu") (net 2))
 (segment (start 147.1705 56.66) (end 146.0815 57.749) (width 1) (layer "B.Cu") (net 2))
 (segment (start 146.931476 65.731) (end 149.633524 65.731) (width 1) (layer "B.Cu") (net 2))
 (segment (start 151.684499 63.680025) (end 151.684499 25.081505) (width 1) (layer "B.Cu") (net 2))
 (segment (start 127 32.26) (end 127.09694 32.26) (width 1) (layer "F.Cu") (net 28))
 (segment (start 124.46 50.8) (end 132.08 58.42) (width 1) (layer "F.Cu") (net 28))
 (segment (start 129.54 34.70306) (end 129.54 45.72) (width 1) (layer "F.Cu") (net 28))
 (segment (start 129.54 45.72) (end 124.46 50.8) (width 1) (layer "F.Cu") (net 28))
 (segment (start 127.09694 32.26) (end 129.54 34.70306) (width 1) (layer "F.Cu") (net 28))
 (segment (start 128.201 35.06253) (end 128.201 44.519) (width 1) (layer "F.Cu") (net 25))
 (segment (start 121.92 50.8) (end 121.92 60.96) (width 1) (layer "F.Cu") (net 25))
 (segment (start 127 33.91) (end 127.04847 33.91) (width 1) (layer "F.Cu") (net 25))
 (segment (start 121.92 60.96) (end 132.08 71.12) (width 1) (layer "F.Cu") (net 25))
 (segment (start 127.04847 33.91) (end 128.201 35.06253) (width 1) (layer "F.Cu") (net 25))
 (segment (start 128.201 44.519) (end 121.92 50.8) (width 1) (layer "F.Cu") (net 25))
 (segment (start 127 35.56) (end 127 43.18) (width 1) (layer "F.Cu") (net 7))
 (segment (start 127 43.18) (end 116.84 53.34) (width 1) (layer "F.Cu") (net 7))
 (segment (start 149.633524 24.729) (end 146.931476 24.729) (width 1) (layer "B.Cu") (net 1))
 (segment (start 148.2825 59.2) (end 148.544524 59.2) (width 1) (layer "B.Cu") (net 1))
 (segment (start 150.4835 57.261024) (end 150.4835 25.578976) (width 1) (layer "B.Cu") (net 1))
 (segment (start 150.4835 25.578976) (end 149.633524 24.729) (width 1) (layer "B.Cu") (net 1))
 (segment (start 144.78 26.880476) (end 144.78 50.8) (width 1) (layer "B.Cu") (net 1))
 (segment (start 148.544524 59.2) (end 150.4835 57.261024) (width 1) (layer "B.Cu") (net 1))
 (segment (start 137.16 55.88) (end 132.08 50.8) (width 1) (layer "B.Cu") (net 1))
 (segment (start 137.16 58.42) (end 137.16 55.88) (width 1) (layer "B.Cu") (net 1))
 (segment (start 144.78 50.8) (end 137.16 58.42) (width 1) (layer "B.Cu") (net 1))
 (segment (start 146.931476 24.729) (end 144.78 26.880476) (width 1) (layer "B.Cu") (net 1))
 (segment (start 114.3 55.88) (end 116.84 58.42) (width 1) (layer "B.Cu") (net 9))
 (segment (start 68.58 55.88) (end 114.3 55.88) (width 1) (layer "B.Cu") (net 9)))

